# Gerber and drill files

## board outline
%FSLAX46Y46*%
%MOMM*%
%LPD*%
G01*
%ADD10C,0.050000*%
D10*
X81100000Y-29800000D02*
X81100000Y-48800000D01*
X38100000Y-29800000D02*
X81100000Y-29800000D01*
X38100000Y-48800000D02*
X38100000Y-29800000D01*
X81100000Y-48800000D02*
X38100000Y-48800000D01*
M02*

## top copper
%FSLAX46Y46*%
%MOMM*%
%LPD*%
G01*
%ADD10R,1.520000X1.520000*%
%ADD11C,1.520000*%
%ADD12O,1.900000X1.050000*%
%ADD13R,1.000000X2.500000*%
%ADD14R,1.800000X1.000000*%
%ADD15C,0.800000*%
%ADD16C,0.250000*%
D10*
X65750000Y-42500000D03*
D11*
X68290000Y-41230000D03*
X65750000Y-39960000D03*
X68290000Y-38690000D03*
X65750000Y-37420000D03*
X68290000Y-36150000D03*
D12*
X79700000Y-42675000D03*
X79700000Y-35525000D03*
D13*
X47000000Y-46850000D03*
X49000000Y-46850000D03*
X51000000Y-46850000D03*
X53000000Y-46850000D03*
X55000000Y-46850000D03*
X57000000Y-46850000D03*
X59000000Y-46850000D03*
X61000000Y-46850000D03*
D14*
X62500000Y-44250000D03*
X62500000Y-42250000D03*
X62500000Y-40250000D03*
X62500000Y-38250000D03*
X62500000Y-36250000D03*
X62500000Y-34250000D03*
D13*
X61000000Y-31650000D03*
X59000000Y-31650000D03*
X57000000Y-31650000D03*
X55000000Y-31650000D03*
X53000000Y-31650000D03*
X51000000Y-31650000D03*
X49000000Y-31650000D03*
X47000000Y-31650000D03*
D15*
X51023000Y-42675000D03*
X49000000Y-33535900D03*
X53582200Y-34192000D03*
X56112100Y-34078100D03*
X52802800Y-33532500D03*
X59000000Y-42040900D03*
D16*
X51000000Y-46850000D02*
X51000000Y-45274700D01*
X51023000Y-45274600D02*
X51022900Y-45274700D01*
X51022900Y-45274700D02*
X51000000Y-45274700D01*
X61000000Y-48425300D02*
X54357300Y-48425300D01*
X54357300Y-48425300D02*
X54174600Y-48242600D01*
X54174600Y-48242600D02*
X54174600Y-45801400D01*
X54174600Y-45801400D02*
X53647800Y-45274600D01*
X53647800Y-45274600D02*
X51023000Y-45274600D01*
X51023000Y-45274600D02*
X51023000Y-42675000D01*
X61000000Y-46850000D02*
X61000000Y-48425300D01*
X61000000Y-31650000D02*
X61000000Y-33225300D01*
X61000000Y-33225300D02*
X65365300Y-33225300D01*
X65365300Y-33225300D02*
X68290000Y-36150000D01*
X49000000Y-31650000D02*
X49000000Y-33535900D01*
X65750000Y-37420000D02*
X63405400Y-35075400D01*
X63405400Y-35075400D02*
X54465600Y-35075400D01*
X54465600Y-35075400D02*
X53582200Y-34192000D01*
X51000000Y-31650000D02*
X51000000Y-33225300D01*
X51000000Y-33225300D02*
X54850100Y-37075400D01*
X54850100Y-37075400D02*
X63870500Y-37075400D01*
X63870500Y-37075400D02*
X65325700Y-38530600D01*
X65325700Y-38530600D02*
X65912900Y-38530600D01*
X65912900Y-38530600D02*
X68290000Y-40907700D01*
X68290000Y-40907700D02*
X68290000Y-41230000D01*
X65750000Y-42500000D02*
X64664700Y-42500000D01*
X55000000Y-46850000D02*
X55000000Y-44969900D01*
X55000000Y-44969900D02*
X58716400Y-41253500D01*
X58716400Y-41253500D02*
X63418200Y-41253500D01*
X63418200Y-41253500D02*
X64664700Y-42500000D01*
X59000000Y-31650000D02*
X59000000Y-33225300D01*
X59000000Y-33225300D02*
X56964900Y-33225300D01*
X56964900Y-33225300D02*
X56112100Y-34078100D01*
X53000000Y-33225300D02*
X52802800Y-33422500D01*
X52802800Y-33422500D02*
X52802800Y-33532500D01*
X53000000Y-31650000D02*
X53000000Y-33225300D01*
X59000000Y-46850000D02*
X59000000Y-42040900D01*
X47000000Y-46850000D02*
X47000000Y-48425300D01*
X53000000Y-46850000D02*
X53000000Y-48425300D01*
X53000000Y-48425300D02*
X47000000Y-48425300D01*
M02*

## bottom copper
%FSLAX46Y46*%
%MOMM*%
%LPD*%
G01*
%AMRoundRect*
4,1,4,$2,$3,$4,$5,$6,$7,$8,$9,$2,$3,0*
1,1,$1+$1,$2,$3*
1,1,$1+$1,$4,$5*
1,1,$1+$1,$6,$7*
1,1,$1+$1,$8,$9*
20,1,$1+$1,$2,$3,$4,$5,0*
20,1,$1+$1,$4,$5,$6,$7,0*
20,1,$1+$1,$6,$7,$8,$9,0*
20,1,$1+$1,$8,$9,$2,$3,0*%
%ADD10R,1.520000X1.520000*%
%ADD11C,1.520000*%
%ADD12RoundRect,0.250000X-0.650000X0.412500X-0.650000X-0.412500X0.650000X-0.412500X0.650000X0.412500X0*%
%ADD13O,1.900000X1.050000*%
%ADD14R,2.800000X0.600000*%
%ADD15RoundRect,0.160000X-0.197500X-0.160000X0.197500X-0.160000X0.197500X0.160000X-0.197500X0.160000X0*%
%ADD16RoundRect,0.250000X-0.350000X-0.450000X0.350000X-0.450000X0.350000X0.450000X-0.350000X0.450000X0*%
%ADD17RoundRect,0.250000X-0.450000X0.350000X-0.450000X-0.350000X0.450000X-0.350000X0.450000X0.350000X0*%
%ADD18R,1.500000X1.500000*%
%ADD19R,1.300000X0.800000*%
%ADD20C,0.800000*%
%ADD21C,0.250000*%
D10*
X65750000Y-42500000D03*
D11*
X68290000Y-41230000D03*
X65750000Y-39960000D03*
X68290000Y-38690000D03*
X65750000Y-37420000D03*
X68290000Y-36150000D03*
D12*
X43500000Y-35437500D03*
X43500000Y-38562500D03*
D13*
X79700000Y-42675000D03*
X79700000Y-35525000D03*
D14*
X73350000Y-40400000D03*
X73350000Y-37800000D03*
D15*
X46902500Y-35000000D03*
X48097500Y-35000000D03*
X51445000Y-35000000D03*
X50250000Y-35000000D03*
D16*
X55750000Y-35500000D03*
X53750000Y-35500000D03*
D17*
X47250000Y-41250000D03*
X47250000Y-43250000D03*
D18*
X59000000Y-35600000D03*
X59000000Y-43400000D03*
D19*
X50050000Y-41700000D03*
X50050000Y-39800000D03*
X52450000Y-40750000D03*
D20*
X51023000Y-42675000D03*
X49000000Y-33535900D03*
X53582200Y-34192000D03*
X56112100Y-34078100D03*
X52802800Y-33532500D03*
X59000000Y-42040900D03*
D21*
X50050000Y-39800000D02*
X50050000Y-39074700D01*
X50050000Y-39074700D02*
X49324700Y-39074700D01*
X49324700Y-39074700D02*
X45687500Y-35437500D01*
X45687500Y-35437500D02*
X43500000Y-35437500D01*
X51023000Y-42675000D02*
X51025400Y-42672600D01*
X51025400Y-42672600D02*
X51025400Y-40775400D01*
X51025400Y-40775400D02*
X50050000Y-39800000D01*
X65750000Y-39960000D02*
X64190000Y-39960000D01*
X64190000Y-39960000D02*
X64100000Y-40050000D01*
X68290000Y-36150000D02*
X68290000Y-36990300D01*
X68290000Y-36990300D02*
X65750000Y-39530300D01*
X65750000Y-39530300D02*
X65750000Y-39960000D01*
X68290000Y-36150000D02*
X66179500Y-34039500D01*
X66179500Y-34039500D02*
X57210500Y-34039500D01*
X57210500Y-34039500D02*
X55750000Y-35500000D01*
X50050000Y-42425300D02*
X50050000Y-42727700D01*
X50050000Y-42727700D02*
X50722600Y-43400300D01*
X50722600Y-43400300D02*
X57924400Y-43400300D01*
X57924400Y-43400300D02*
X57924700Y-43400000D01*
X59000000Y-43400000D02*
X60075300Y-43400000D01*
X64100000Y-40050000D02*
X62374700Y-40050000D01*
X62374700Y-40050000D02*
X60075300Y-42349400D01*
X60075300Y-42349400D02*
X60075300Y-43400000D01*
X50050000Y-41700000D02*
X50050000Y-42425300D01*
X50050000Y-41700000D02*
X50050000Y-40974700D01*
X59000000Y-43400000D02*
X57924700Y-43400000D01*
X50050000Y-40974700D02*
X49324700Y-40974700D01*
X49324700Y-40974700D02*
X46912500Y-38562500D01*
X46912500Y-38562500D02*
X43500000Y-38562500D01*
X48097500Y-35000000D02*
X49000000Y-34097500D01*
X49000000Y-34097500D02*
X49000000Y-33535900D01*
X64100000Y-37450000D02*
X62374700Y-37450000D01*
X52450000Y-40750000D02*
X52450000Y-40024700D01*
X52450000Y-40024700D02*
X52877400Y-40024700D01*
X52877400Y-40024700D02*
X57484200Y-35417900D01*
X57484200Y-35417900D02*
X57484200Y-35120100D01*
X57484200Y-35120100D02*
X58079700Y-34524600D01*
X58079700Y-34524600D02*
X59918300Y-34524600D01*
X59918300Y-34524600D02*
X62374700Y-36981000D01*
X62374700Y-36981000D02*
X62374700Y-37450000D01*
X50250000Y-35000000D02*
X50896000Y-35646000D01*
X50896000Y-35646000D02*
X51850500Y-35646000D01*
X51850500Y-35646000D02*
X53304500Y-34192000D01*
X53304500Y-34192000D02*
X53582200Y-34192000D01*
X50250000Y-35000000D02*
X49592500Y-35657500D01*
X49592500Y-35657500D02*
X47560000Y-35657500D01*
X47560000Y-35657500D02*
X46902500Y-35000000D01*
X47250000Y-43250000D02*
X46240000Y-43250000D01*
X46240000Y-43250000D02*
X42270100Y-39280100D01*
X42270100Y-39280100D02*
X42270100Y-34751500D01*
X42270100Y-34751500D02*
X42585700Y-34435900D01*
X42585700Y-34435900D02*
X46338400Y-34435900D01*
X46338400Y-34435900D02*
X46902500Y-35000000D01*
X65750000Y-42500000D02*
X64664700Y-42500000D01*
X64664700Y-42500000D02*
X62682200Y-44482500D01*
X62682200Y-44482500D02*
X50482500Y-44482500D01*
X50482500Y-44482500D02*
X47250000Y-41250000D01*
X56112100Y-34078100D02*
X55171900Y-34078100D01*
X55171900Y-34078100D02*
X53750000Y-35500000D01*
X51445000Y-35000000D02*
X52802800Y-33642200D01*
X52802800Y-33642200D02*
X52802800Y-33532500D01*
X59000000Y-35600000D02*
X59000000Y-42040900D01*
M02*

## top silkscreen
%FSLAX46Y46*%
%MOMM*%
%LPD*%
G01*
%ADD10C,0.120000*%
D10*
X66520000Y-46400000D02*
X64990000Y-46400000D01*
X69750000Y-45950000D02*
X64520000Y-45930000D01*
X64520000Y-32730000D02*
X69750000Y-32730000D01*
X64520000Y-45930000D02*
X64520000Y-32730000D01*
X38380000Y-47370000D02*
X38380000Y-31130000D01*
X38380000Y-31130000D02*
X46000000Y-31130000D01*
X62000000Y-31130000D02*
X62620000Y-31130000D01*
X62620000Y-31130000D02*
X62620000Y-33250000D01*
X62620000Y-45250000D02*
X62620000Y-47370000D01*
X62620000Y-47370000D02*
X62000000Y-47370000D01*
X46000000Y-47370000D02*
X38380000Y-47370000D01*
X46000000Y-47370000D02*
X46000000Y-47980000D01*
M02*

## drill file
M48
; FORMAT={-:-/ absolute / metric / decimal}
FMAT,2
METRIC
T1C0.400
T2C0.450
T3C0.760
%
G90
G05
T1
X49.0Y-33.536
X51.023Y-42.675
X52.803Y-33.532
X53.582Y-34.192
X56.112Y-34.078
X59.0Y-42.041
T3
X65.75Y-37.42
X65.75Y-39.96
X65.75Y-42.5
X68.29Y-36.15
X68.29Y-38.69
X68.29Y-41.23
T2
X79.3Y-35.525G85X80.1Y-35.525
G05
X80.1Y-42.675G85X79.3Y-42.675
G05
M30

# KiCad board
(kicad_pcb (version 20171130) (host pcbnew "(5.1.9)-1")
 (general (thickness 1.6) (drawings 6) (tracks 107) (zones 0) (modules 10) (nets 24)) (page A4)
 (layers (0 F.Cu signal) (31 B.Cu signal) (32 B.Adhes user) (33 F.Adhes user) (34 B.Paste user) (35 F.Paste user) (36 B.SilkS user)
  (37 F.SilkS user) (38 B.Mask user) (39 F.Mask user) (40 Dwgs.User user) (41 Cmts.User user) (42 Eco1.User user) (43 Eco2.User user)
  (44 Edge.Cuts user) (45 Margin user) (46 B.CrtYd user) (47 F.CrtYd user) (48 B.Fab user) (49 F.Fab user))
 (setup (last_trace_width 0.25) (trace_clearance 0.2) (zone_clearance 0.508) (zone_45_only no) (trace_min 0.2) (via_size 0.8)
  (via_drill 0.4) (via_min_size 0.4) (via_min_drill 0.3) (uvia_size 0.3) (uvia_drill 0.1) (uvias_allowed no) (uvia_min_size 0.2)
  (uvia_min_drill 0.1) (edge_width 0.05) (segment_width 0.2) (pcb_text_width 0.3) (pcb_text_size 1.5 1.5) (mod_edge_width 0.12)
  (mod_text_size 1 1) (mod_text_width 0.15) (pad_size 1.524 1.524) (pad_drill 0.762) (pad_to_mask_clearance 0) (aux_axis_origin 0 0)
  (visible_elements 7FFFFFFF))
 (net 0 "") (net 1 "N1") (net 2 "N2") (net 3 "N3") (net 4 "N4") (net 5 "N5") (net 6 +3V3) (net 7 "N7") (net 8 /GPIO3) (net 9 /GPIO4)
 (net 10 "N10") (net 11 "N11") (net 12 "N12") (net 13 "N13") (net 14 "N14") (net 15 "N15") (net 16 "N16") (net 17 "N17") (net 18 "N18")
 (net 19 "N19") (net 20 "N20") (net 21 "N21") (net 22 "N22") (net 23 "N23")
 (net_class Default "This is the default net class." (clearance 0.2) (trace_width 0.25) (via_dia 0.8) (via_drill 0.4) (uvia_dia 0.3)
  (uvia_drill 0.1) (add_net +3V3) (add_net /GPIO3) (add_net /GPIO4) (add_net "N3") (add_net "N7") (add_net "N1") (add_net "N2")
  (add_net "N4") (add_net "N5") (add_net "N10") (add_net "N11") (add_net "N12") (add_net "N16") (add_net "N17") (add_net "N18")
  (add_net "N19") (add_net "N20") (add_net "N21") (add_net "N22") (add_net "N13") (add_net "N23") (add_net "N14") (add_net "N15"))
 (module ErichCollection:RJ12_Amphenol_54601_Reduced (layer F.Cu) (at 65.75 42.5 90)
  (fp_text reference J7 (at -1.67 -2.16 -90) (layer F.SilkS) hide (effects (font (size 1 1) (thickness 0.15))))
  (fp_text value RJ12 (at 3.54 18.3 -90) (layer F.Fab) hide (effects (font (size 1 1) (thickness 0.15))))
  (fp_line (start -3.9 0.77) (end -3.9 -0.76) (layer F.SilkS) (width 0.12))
  (fp_line (start -3.45 4) (end -3.43 -1.23) (layer F.SilkS) (width 0.12))
  (fp_line (start 9.77 -1.23) (end 9.77 4) (layer F.SilkS) (width 0.12))
  (fp_line (start -3.43 -1.23) (end 9.77 -1.23) (layer F.SilkS) (width 0.12))
  (pad 1 thru_hole rect (at 0 0 90) (size 1.52 1.52) (drill 0.76) (layers *.Cu *.Mask) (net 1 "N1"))
  (pad 2 thru_hole circle (at 1.27 2.54 90) (size 1.52 1.52) (drill 0.76) (layers *.Cu *.Mask) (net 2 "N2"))
  (pad 3 thru_hole circle (at 2.54 0 90) (size 1.52 1.52) (drill 0.76) (layers *.Cu *.Mask) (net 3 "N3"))
  (pad 4 thru_hole circle (at 3.81 2.54 90) (size 1.52 1.52) (drill 0.76) (layers *.Cu *.Mask) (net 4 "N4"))
  (pad 5 thru_hole circle (at 5.08 0 90) (size 1.52 1.52) (drill 0.76) (layers *.Cu *.Mask) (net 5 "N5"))
  (pad 6 thru_hole circle (at 6.35 2.54 90) (size 1.52 1.52) (drill 0.76) (layers *.Cu *.Mask) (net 3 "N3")))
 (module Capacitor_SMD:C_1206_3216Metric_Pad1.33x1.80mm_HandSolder (layer B.Cu) (at 43.5 37 270)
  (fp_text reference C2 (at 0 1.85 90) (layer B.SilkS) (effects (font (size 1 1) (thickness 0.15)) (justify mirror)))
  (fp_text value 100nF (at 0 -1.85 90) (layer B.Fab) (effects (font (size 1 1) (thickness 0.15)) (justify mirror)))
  (pad 1 smd roundrect (at -1.5625 0 270) (size 1.325 1.8) (layers B.Cu B.Paste B.Mask) (roundrect_rratio 0.188679) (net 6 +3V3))
  (pad 2 smd roundrect (at 1.5625 0 270) (size 1.325 1.8) (layers B.Cu B.Paste B.Mask) (roundrect_rratio 0.188679) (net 3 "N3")))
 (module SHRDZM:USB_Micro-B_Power (layer B.Cu) (at 78.5 39.1 270)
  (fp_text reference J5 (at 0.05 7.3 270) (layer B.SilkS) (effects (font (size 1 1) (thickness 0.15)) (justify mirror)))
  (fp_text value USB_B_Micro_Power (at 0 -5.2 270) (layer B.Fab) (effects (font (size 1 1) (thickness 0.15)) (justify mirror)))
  (pad "" thru_hole oval (at 3.575 -1.2 270) (size 1.05 1.9) (drill oval 0.45 1.25) (layers *.Cu *.Mask))
  (pad "" thru_hole oval (at -3.575 -1.2 90) (size 1.05 1.9) (drill oval 0.45 1.25) (layers *.Cu *.Mask))
  (pad 5 smd rect (at 1.3 5.15 270) (size 0.6 2.8) (layers B.Cu B.Paste B.Mask) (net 3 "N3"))
  (pad 1 smd rect (at -1.3 5.15 270) (size 0.6 2.8) (layers B.Cu B.Paste B.Mask) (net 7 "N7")))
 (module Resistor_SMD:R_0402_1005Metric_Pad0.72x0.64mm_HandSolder (layer B.Cu) (at 47.5 35)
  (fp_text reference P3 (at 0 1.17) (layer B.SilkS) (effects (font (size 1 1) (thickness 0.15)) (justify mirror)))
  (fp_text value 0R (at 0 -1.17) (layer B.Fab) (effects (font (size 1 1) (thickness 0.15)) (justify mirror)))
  (pad 1 smd roundrect (at -0.5975 0) (size 0.715 0.64) (layers B.Cu B.Paste B.Mask) (roundrect_rratio 0.25) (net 5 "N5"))
  (pad 2 smd roundrect (at 0.5975 0) (size 0.715 0.64) (layers B.Cu B.Paste B.Mask) (roundrect_rratio 0.25) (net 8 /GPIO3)))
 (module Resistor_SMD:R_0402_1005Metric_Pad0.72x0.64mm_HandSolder (layer B.Cu) (at 50.8475 35)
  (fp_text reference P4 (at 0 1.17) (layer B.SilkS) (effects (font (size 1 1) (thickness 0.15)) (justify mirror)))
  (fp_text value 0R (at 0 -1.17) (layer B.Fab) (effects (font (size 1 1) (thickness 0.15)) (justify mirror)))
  (pad 2 smd roundrect (at 0.5975 0) (size 0.715 0.64) (layers B.Cu B.Paste B.Mask) (roundrect_rratio 0.25) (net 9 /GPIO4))
  (pad 1 smd roundrect (at -0.5975 0) (size 0.715 0.64) (layers B.Cu B.Paste B.Mask) (roundrect_rratio 0.25) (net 5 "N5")))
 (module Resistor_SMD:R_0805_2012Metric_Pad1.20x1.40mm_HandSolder (layer B.Cu) (at 54.75 35.5)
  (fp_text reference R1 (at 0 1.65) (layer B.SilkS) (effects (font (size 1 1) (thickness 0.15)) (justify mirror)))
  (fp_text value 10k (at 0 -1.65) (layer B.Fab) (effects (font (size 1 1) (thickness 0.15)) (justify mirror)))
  (pad 2 smd roundrect (at 1 0) (size 1.2 1.4) (layers B.Cu B.Paste B.Mask) (roundrect_rratio 0.208333) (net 3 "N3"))
  (pad 1 smd roundrect (at -1 0) (size 1.2 1.4) (layers B.Cu B.Paste B.Mask) (roundrect_rratio 0.208333) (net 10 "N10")))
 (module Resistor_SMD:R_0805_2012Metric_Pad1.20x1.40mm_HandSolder (layer B.Cu) (at 47.25 42.25 270)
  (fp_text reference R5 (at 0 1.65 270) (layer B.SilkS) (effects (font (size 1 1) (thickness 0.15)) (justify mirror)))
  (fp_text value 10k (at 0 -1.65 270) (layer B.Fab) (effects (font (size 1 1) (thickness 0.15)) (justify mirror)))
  (pad 1 smd roundrect (at -1 0 270) (size 1.2 1.4) (layers B.Cu B.Paste B.Mask) (roundrect_rratio 0.208333) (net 1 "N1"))
  (pad 2 smd roundrect (at 1 0 270) (size 1.2 1.4) (layers B.Cu B.Paste B.Mask) (roundrect_rratio 0.208333) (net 5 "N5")))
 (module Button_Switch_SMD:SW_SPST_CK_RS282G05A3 (layer B.Cu) (at 59 39.5 270)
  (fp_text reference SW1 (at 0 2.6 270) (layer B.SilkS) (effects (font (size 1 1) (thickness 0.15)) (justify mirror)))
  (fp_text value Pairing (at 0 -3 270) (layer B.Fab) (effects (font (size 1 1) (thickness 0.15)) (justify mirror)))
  (pad 1 smd rect (at -3.9 0 270) (size 1.5 1.5) (layers B.Cu B.Paste B.Mask) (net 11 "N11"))
  (pad 2 smd rect (at 3.9 0 270) (size 1.5 1.5) (layers B.Cu B.Paste B.Mask) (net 3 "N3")))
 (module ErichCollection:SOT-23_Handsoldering (layer B.Cu) (at 51.25 40.75)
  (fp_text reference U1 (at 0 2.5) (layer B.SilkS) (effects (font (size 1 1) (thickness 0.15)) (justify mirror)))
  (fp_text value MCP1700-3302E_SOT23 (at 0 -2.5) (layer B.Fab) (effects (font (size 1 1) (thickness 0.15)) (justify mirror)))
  (pad 1 smd rect (at -1.2 0.95) (size 1.3 0.8) (layers B.Cu B.Paste B.Mask) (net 3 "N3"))
  (pad 2 smd rect (at -1.2 -0.95) (size 1.3 0.8) (layers B.Cu B.Paste B.Mask) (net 6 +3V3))
  (pad 3 smd rect (at 1.2 0) (size 1.3 0.8) (layers B.Cu B.Paste B.Mask) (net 7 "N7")))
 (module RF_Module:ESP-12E (layer F.Cu) (at 50.5 39.25 90)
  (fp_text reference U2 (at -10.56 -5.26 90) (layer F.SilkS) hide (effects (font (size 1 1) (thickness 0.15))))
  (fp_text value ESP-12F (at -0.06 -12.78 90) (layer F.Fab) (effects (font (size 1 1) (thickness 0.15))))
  (fp_line (start -8.12 -12.12) (end 8.12 -12.12) (layer F.SilkS) (width 0.12))
  (fp_line (start 8.12 -12.12) (end 8.12 -4.5) (layer F.SilkS) (width 0.12))
  (fp_line (start 8.12 11.5) (end 8.12 12.12) (layer F.SilkS) (width 0.12))
  (fp_line (start 8.12 12.12) (end 6 12.12) (layer F.SilkS) (width 0.12))
  (fp_line (start -6 12.12) (end -8.12 12.12) (layer F.SilkS) (width 0.12))
  (fp_line (start -8.12 12.12) (end -8.12 11.5) (layer F.SilkS) (width 0.12))
  (fp_line (start -8.12 -4.5) (end -8.12 -12.12) (layer F.SilkS) (width 0.12))
  (fp_line (start -8.12 -4.5) (end -8.73 -4.5) (layer F.SilkS) (width 0.12))
  (pad 1 smd rect (at -7.6 -3.5 90) (size 2.5 1) (layers F.Cu F.Paste F.Mask) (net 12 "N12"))
  (pad 2 smd rect (at -7.6 -1.5 90) (size 2.5 1) (layers F.Cu F.Paste F.Mask) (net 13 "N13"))
  (pad 3 smd rect (at -7.6 0.5 90) (size 2.5 1) (layers F.Cu F.Paste F.Mask) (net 6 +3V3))
  (pad 4 smd rect (at -7.6 2.5 90) (size 2.5 1) (layers F.Cu F.Paste F.Mask) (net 12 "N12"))
  (pad 5 smd rect (at -7.6 4.5 90) (size 2.5 1) (layers F.Cu F.Paste F.Mask) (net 1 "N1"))
  (pad 6 smd rect (at -7.6 6.5 90) (size 2.5 1) (layers F.Cu F.Paste F.Mask) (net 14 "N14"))
  (pad 7 smd rect (at -7.6 8.5 90) (size 2.5 1) (layers F.Cu F.Paste F.Mask) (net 11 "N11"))
  (pad 8 smd rect (at -7.6 10.5 90) (size 2.5 1) (layers F.Cu F.Paste F.Mask) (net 6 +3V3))
  (pad 9 smd rect (at -5 12 90) (size 1 1.8) (layers F.Cu F.Paste F.Mask) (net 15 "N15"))
  (pad 10 smd rect (at -3 12 90) (size 1 1.8) (layers F.Cu F.Paste F.Mask) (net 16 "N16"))
  (pad 11 smd rect (at -1 12 90) (size 1 1.8) (layers F.Cu F.Paste F.Mask) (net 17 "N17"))
  (pad 12 smd rect (at 1 12 90) (size 1 1.8) (layers F.Cu F.Paste F.Mask) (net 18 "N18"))
  (pad 13 smd rect (at 3 12 90) (size 1 1.8) (layers F.Cu F.Paste F.Mask) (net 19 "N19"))
  (pad 14 smd rect (at 5 12 90) (size 1 1.8) (layers F.Cu F.Paste F.Mask) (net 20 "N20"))
  (pad 15 smd rect (at 7.6 10.5 90) (size 2.5 1) (layers F.Cu F.Paste F.Mask) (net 3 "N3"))
  (pad 16 smd rect (at 7.6 8.5 90) (size 2.5 1) (layers F.Cu F.Paste F.Mask) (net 10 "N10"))
  (pad 17 smd rect (at 7.6 6.5 90) (size 2.5 1) (layers F.Cu F.Paste F.Mask) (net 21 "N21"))
  (pad 18 smd rect (at 7.6 4.5 90) (size 2.5 1) (layers F.Cu F.Paste F.Mask) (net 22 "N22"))
  (pad 19 smd rect (at 7.6 2.5 90) (size 2.5 1) (layers F.Cu F.Paste F.Mask) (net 9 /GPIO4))
  (pad 20 smd rect (at 7.6 0.5 90) (size 2.5 1) (layers F.Cu F.Paste F.Mask) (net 2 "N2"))
  (pad 21 smd rect (at 7.6 -1.5 90) (size 2.5 1) (layers F.Cu F.Paste F.Mask) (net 8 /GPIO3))
  (pad 22 smd rect (at 7.6 -3.5 90) (size 2.5 1) (layers F.Cu F.Paste F.Mask) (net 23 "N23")))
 (gr_line (start 81.1 29.8) (end 81.1 48.8) (layer Edge.Cuts) (width 0.05))
 (gr_line (start 38.1 29.8) (end 81.1 29.8) (layer Edge.Cuts) (width 0.05))
 (gr_line (start 38.1 48.8) (end 38.1 29.8) (layer Edge.Cuts) (width 0.05))
 (gr_line (start 81.1 48.8) (end 38.1 48.8) (layer Edge.Cuts) (width 0.05))
 (segment (start 50.05 39.8) (end 50.05 39.0747) (width 0.25) (layer B.Cu) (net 6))
 (segment (start 50.05 39.0747) (end 49.3247 39.0747) (width 0.25) (layer B.Cu) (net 6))
 (segment (start 49.3247 39.0747) (end 45.6875 35.4375) (width 0.25) (layer B.Cu) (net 6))
 (segment (start 45.6875 35.4375) (end 43.5 35.4375) (width 0.25) (layer B.Cu) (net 6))
 (segment (start 51.023 42.675) (end 51.0254 42.6726) (width 0.25) (layer B.Cu) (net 6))
 (segment (start 51.0254 42.6726) (end 51.0254 40.7754) (width 0.25) (layer B.Cu) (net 6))
 (segment (start 51.0254 40.7754) (end 50.05 39.8) (width 0.25) (layer B.Cu) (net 6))
 (segment (start 51 46.85) (end 51 45.2747) (width 0.25) (layer F.Cu) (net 6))
 (segment (start 51.023 45.2746) (end 51.0229 45.2747) (width 0.25) (layer F.Cu) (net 6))
 (segment (start 51.0229 45.2747) (end 51 45.2747) (width 0.25) (layer F.Cu) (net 6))
 (segment (start 61 48.4253) (end 54.3573 48.4253) (width 0.25) (layer F.Cu) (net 6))
 (segment (start 54.3573 48.4253) (end 54.1746 48.2426) (width 0.25) (layer F.Cu) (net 6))
 (segment (start 54.1746 48.2426) (end 54.1746 45.8014) (width 0.25) (layer F.Cu) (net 6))
 (segment (start 54.1746 45.8014) (end 53.6478 45.2746) (width 0.25) (layer F.Cu) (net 6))
 (segment (start 53.6478 45.2746) (end 51.023 45.2746) (width 0.25) (layer F.Cu) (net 6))
 (segment (start 51.023 45.2746) (end 51.023 42.675) (width 0.25) (layer F.Cu) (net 6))
 (segment (start 61 46.85) (end 61 48.4253) (width 0.25) (layer F.Cu) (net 6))
 (via (at 51.023 42.675) (size 0.8) (layers F.Cu B.Cu) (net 6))
 (segment (start 65.75 39.96) (end 64.19 39.96) (width 0.25) (layer B.Cu) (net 3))
 (segment (start 64.19 39.96) (end 64.1 40.05) (width 0.25) (layer B.Cu) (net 3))
 (segment (start 68.29 36.15) (end 68.29 36.9903) (width 0.25) (layer B.Cu) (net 3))
 (segment (start 68.29 36.9903) (end 65.75 39.5303) (width 0.25) (layer B.Cu) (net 3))
 (segment (start 65.75 39.5303) (end 65.75 39.96) (width 0.25) (layer B.Cu) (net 3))
 (segment (start 68.29 36.15) (end 66.1795 34.0395) (width 0.25) (layer B.Cu) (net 3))
 (segment (start 66.1795 34.0395) (end 57.2105 34.0395) (width 0.25) (layer B.Cu) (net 3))
 (segment (start 57.2105 34.0395) (end 55.75 35.5) (width 0.25) (layer B.Cu) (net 3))
 (segment (start 50.05 42.4253) (end 50.05 42.7277) (width 0.25) (layer B.Cu) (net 3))
 (segment (start 50.05 42.7277) (end 50.7226 43.4003) (width 0.25) (layer B.Cu) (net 3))
 (segment (start 50.7226 43.4003) (end 57.9244 43.4003) (width 0.25) (layer B.Cu) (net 3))
 (segment (start 57.9244 43.4003) (end 57.9247 43.4) (width 0.25) (layer B.Cu) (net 3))
 (segment (start 61 31.65) (end 61 33.2253) (width 0.25) (layer F.Cu) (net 3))
 (segment (start 61 33.2253) (end 65.3653 33.2253) (width 0.25) (layer F.Cu) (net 3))
 (segment (start 65.3653 33.2253) (end 68.29 36.15) (width 0.25) (layer F.Cu) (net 3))
 (segment (start 59 43.4) (end 60.0753 43.4) (width 0.25) (layer B.Cu) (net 3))
 (segment (start 64.1 40.05) (end 62.3747 40.05) (width 0.25) (layer B.Cu) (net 3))
 (segment (start 62.3747 40.05) (end 60.0753 42.3494) (width 0.25) (layer B.Cu) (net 3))
 (segment (start 60.0753 42.3494) (end 60.0753 43.4) (width 0.25) (layer B.Cu) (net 3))
 (segment (start 50.05 41.7) (end 50.05 42.4253) (width 0.25) (layer B.Cu) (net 3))
 (segment (start 50.05 41.7) (end 50.05 40.9747) (width 0.25) (layer B.Cu) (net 3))
 (segment (start 59 43.4) (end 57.9247 43.4) (width 0.25) (layer B.Cu) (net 3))
 (segment (start 50.05 40.9747) (end 49.3247 40.9747) (width 0.25) (layer B.Cu) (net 3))
 (segment (start 49.3247 40.9747) (end 46.9125 38.5625) (width 0.25) (layer B.Cu) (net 3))
 (segment (start 46.9125 38.5625) (end 43.5 38.5625) (width 0.25) (layer B.Cu) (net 3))
 (segment (start 49 31.65) (end 49 33.5359) (width 0.25) (layer F.Cu) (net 8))
 (segment (start 48.0975 35) (end 49 34.0975) (width 0.25) (layer B.Cu) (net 8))
 (segment (start 49 34.0975) (end 49 33.5359) (width 0.25) (layer B.Cu) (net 8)) (via (at 49 33.5359) (size 0.8) (layers F.Cu B.Cu) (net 8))
 (segment (start 64.1 37.45) (end 62.3747 37.45) (width 0.25) (layer B.Cu) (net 7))
 (segment (start 52.45 40.75) (end 52.45 40.0247) (width 0.25) (layer B.Cu) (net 7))
 (segment (start 52.45 40.0247) (end 52.8774 40.0247) (width 0.25) (layer B.Cu) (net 7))
 (segment (start 52.8774 40.0247) (end 57.4842 35.4179) (width 0.25) (layer B.Cu) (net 7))
 (segment (start 57.4842 35.4179) (end 57.4842 35.1201) (width 0.25) (layer B.Cu) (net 7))
 (segment (start 57.4842 35.1201) (end 58.0797 34.5246) (width 0.25) (layer B.Cu) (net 7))
 (segment (start 58.0797 34.5246) (end 59.9183 34.5246) (width 0.25) (layer B.Cu) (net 7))
 (segment (start 59.9183 34.5246) (end 62.3747 36.981) (width 0.25) (layer B.Cu) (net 7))
 (segment (start 62.3747 36.981) (end 62.3747 37.45) (width 0.25) (layer B.Cu) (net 7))
 (segment (start 50.25 35) (end 50.896 35.646) (width 0.25) (layer B.Cu) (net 5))
 (segment (start 50.896 35.646) (end 51.8505 35.646) (width 0.25) (layer B.Cu) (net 5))
 (segment (start 51.8505 35.646) (end 53.3045 34.192) (width 0.25) (layer B.Cu) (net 5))
 (segment (start 53.3045 34.192) (end 53.5822 34.192) (width 0.25) (layer B.Cu) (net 5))
 (segment (start 50.25 35) (end 49.5925 35.6575) (width 0.25) (layer B.Cu) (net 5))
 (segment (start 49.5925 35.6575) (end 47.56 35.6575) (width 0.25) (layer B.Cu) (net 5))
 (segment (start 47.56 35.6575) (end 46.9025 35) (width 0.25) (layer B.Cu) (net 5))
 (segment (start 47.25 43.25) (end 46.24 43.25) (width 0.25) (layer B.Cu) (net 5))
 (segment (start 46.24 43.25) (end 42.2701 39.2801) (width 0.25) (layer B.Cu) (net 5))
 (segment (start 42.2701 39.2801) (end 42.2701 34.7515) (width 0.25) (layer B.Cu) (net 5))
 (segment (start 42.2701 34.7515) (end 42.5857 34.4359) (width 0.25) (layer B.Cu) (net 5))
 (segment (start 42.5857 34.4359) (end 46.3384 34.4359) (width 0.25) (layer B.Cu) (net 5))
 (segment (start 46.3384 34.4359) (end 46.9025 35) (width 0.25) (layer B.Cu) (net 5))
 (segment (start 65.75 37.42) (end 63.4054 35.0754) (width 0.25) (layer F.Cu) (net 5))
 (segment (start 63.4054 35.0754) (end 54.4656 35.0754) (width 0.25) (layer F.Cu) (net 5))
 (segment (start 54.4656 35.0754) (end 53.5822 34.192) (width 0.25) (layer F.Cu) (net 5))
 (via (at 53.5822 34.192) (size 0.8) (layers F.Cu B.Cu) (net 5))
 (segment (start 51 31.65) (end 51 33.2253) (width 0.25) (layer F.Cu) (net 2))
 (segment (start 51 33.2253) (end 54.8501 37.0754) (width 0.25) (layer F.Cu) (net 2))
 (segment (start 54.8501 37.0754) (end 63.8705 37.0754) (width 0.25) (layer F.Cu) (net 2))
 (segment (start 63.8705 37.0754) (end 65.3257 38.5306) (width 0.25) (layer F.Cu) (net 2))
 (segment (start 65.3257 38.5306) (end 65.9129 38.5306) (width 0.25) (layer F.Cu) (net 2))
 (segment (start 65.9129 38.5306) (end 68.29 40.9077) (width 0.25) (layer F.Cu) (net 2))
 (segment (start 68.29 40.9077) (end 68.29 41.23) (width 0.25) (layer F.Cu) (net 2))
 (segment (start 65.75 42.5) (end 64.6647 42.5) (width 0.25) (layer B.Cu) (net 1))
 (segment (start 64.6647 42.5) (end 62.6822 44.4825) (width 0.25) (layer B.Cu) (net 1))
 (segment (start 62.6822 44.4825) (end 50.4825 44.4825) (width 0.25) (layer B.Cu) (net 1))
 (segment (start 50.4825 44.4825) (end 47.25 41.25) (width 0.25) (layer B.Cu) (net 1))
 (segment (start 65.75 42.5) (end 64.6647 42.5) (width 0.25) (layer F.Cu) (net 1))
 (segment (start 55 46.85) (end 55 44.9699) (width 0.25) (layer F.Cu) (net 1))
 (segment (start 55 44.9699) (end 58.7164 41.2535) (width 0.25) (layer F.Cu) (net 1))
 (segment (start 58.7164 41.2535) (end 63.4182 41.2535) (width 0.25) (layer F.Cu) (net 1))
 (segment (start 63.4182 41.2535) (end 64.6647 42.5) (width 0.25) (layer F.Cu) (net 1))
 (segment (start 59 31.65) (end 59 33.2253) (width 0.25) (layer F.Cu) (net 10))
 (segment (start 56.1121 34.0781) (end 55.1719 34.0781) (width 0.25) (layer B.Cu) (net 10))
 (segment (start 55.1719 34.0781) (end 53.75 35.5) (width 0.25) (layer B.Cu) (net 10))
 (segment (start 59 33.2253) (end 56.9649 33.2253) (width 0.25) (layer F.Cu) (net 10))
 (segment (start 56.9649 33.2253) (end 56.1121 34.0781) (width 0.25) (layer F.Cu) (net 10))
 (via (at 56.1121 34.0781) (size 0.8) (layers F.Cu B.Cu) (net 10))
 (segment (start 53 33.2253) (end 52.8028 33.4225) (width 0.25) (layer F.Cu) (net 9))
 (segment (start 52.8028 33.4225) (end 52.8028 33.5325) (width 0.25) (layer F.Cu) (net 9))
 (segment (start 51.445 35) (end 52.8028 33.6422) (width 0.25) (layer B.Cu) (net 9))
 (segment (start 52.8028 33.6422) (end 52.8028 33.5325) (width 0.25) (layer B.Cu) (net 9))
 (segment (start 53 31.65) (end 53 33.2253) (width 0.25) (layer F.Cu) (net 9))
 (via (at 52.8028 33.5325) (size 0.8) (layers F.Cu B.Cu) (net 9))
 (segment (start 59 46.85) (end 59 42.0409) (width 0.25) (layer F.Cu) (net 11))
 (segment (start 59 35.6) (end 59 42.0409) (width 0.25) (layer B.Cu) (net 11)) (via (at 59 42.0409) (size 0.8) (layers F.Cu B.Cu) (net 11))
 (segment (start 47 46.85) (end 47 48.4253) (width 0.25) (layer F.Cu) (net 12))
 (segment (start 53 46.85) (end 53 48.4253) (width 0.25) (layer F.Cu) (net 12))
 (segment (start 53 48.4253) (end 47 48.4253) (width 0.25) (layer F.Cu) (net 12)))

